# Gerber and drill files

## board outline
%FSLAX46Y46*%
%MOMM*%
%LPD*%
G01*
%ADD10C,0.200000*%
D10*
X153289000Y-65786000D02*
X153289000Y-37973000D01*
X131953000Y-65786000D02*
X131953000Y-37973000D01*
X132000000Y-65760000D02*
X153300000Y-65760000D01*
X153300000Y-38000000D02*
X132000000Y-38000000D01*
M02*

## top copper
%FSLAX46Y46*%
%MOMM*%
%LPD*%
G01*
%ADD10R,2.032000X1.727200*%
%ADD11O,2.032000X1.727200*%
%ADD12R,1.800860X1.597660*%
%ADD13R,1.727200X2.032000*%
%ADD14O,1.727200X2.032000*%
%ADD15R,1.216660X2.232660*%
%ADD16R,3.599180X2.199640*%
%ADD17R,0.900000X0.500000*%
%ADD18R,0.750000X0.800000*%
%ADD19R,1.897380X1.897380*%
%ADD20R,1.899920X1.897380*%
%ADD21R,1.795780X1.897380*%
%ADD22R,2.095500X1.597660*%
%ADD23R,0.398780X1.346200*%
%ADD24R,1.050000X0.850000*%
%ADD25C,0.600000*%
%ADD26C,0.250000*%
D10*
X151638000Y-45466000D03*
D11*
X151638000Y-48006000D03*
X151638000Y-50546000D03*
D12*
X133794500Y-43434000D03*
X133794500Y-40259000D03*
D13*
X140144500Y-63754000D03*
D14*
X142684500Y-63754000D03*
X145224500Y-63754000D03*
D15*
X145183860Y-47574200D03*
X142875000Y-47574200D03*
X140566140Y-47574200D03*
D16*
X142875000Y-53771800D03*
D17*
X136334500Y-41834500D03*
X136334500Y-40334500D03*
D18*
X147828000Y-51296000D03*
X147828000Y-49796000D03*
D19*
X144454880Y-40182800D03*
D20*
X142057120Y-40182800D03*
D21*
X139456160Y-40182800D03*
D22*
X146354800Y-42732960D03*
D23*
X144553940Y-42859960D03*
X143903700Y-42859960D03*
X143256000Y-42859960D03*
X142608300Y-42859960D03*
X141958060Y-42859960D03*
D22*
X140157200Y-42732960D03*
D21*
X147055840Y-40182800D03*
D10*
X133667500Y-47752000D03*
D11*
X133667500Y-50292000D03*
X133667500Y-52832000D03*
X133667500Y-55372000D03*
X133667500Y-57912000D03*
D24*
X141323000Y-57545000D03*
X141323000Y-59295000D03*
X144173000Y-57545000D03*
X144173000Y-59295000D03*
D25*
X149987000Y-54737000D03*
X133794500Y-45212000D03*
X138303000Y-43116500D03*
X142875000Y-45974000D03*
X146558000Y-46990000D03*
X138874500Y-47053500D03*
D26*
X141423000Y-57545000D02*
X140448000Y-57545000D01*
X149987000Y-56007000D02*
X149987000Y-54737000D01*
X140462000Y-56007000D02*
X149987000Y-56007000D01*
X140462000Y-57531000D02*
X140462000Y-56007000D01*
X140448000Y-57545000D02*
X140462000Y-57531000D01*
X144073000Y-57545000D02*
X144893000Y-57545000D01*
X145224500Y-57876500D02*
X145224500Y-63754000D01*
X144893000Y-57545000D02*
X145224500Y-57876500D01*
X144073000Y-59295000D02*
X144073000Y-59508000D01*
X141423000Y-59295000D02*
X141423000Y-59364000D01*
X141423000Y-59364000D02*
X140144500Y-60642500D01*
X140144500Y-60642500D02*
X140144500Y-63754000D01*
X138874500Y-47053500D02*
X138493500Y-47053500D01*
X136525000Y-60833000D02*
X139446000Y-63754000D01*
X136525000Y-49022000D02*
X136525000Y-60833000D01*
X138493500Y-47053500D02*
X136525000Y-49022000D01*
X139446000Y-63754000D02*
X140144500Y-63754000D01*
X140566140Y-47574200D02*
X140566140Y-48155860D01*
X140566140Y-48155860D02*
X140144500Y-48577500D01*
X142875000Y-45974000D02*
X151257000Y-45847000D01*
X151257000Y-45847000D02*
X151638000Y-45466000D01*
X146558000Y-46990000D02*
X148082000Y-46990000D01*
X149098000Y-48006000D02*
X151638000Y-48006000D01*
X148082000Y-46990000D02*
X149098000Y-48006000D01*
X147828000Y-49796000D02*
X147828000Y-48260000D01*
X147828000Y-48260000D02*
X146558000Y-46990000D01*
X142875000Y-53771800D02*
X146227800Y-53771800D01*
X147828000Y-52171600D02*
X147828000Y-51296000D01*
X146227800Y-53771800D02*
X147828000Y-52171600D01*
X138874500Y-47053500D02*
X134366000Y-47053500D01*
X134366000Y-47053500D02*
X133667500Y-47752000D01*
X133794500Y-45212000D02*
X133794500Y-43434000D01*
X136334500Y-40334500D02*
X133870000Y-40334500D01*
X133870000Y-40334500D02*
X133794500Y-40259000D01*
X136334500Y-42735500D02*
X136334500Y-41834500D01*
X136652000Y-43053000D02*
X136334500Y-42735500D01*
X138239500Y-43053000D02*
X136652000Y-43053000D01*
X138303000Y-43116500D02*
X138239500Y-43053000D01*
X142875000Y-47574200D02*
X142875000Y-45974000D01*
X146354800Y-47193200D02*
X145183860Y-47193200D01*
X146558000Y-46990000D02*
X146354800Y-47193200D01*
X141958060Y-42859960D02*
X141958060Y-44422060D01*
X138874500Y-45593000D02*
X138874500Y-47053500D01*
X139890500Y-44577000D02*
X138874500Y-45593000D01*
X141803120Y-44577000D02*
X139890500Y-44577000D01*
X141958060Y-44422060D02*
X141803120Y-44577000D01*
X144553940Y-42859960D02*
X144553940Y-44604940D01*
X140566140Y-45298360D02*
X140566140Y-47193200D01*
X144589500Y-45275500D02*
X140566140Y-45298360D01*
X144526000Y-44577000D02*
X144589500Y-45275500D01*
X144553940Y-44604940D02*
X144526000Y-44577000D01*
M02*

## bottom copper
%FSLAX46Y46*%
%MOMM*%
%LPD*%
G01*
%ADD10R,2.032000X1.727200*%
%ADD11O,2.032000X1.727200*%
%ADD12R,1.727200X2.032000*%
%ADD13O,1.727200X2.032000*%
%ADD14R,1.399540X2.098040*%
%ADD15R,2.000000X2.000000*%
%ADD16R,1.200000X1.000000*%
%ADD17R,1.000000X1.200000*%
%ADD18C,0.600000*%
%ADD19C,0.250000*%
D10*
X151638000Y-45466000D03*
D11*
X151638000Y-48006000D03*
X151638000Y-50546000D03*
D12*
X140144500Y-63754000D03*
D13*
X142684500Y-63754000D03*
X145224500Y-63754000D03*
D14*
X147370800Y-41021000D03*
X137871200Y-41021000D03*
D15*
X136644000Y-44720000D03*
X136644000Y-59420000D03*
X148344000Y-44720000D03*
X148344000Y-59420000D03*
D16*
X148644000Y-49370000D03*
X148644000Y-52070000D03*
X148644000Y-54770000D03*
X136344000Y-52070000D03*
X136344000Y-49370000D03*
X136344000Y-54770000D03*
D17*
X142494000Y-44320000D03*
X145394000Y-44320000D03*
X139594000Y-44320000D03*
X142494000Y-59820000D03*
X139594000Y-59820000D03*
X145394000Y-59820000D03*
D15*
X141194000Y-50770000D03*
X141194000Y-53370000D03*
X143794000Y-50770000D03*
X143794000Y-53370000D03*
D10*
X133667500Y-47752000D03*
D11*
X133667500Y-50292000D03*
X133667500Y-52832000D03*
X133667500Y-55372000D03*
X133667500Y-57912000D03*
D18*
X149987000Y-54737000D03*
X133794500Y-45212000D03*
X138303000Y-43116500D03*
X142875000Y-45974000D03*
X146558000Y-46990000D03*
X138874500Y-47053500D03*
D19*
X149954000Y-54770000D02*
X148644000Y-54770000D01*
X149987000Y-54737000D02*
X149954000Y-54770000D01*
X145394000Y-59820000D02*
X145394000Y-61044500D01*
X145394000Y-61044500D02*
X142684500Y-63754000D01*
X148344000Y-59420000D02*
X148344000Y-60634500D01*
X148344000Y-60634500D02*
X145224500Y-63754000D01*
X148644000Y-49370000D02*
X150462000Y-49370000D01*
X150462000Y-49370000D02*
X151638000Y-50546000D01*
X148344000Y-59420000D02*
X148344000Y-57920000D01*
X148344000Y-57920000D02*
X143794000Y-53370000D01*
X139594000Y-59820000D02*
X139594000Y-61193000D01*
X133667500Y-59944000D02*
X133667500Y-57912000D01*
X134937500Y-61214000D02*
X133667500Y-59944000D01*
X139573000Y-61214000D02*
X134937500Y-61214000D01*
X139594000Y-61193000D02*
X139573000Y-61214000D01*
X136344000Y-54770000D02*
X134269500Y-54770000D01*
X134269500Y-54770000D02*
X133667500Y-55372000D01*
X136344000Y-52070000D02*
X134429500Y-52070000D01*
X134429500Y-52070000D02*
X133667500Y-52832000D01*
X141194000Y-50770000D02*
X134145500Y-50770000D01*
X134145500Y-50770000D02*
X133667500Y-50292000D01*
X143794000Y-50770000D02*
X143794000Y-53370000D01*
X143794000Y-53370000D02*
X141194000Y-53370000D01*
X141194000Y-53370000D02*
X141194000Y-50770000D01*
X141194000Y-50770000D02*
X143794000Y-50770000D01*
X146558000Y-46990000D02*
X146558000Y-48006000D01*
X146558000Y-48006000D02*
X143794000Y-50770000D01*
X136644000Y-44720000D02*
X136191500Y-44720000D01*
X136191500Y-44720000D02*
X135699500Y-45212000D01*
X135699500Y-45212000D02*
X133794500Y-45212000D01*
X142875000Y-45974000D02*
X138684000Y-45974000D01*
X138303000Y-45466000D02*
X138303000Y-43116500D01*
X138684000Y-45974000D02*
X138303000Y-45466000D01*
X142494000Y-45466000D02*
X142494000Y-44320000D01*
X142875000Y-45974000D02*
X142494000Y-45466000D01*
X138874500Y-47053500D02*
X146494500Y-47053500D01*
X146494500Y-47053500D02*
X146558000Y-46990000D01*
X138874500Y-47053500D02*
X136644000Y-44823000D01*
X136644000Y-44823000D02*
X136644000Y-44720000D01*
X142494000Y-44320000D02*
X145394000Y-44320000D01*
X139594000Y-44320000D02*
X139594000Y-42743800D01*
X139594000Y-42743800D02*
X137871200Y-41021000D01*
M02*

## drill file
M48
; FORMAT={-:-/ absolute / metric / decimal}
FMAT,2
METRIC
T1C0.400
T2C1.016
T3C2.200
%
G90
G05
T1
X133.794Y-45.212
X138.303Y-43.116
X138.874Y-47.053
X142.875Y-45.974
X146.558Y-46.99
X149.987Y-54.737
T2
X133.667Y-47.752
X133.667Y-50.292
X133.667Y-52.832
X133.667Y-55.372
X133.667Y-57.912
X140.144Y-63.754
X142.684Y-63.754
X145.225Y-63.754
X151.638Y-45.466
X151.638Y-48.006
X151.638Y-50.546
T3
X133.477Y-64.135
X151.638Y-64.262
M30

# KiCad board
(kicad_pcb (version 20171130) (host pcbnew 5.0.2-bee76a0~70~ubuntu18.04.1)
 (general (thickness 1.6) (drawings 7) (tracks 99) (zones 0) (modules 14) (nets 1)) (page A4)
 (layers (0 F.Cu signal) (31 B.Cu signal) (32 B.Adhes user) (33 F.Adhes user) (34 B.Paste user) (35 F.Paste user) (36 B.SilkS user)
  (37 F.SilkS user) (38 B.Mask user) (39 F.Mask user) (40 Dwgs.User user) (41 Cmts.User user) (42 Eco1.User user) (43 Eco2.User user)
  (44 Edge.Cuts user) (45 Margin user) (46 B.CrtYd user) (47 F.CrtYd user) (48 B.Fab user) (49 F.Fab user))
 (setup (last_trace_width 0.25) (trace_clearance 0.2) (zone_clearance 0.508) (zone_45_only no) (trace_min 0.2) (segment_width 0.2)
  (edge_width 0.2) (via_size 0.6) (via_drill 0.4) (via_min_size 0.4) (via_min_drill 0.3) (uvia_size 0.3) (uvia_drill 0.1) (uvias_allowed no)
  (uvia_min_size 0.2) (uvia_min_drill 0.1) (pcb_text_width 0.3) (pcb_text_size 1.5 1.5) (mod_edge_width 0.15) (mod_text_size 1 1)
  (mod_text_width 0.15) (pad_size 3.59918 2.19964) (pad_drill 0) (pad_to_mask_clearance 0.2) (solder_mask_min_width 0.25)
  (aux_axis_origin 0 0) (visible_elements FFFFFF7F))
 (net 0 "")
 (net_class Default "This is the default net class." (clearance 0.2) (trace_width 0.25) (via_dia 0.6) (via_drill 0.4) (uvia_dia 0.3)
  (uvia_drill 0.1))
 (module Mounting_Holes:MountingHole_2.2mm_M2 (layer F.Cu) (at 133.477 64.135)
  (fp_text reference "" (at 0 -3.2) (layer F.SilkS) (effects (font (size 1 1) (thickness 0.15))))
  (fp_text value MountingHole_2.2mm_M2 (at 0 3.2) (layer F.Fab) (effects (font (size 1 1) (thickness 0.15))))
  (pad 1 np_thru_hole circle (at 0 0) (size 2.2 2.2) (drill 2.2) (layers *.Cu *.Mask F.SilkS)))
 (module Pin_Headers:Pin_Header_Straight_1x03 (layer F.Cu) (at 151.638 45.466)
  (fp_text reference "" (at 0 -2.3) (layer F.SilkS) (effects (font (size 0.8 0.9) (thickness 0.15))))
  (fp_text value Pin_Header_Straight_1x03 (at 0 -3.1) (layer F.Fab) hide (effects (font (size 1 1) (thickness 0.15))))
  (pad 1 thru_hole rect (at 0 0) (size 2.032 1.7272) (drill 1.016) (layers *.Cu *.Mask F.SilkS))
  (pad 2 thru_hole oval (at 0 2.54) (size 2.032 1.7272) (drill 1.016) (layers *.Cu *.Mask F.SilkS))
  (pad 3 thru_hole oval (at 0 5.08) (size 2.032 1.7272) (drill 1.016) (layers *.Cu *.Mask F.SilkS)))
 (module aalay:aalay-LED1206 (layer F.Cu) (at 133.7945 41.8465 90)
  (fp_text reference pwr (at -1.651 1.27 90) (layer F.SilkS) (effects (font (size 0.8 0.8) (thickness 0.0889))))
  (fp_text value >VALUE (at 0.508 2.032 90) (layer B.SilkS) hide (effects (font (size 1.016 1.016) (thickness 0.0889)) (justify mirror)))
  (pad A smd rect (at -1.5875 0 90) (size 1.59766 1.80086) (layers F.Cu F.Paste F.Mask))
  (pad K smd rect (at 1.5875 0 90) (size 1.59766 1.80086) (layers F.Cu F.Paste F.Mask)))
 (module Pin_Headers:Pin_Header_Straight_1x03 (layer F.Cu) (at 140.1445 63.754 90)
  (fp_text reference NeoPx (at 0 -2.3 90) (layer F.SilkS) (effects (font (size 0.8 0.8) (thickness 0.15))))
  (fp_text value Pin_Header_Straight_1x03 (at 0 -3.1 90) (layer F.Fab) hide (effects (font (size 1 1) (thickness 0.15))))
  (pad 1 thru_hole rect (at 0 0 90) (size 2.032 1.7272) (drill 1.016) (layers *.Cu *.Mask F.SilkS))
  (pad 2 thru_hole oval (at 0 2.54 90) (size 2.032 1.7272) (drill 1.016) (layers *.Cu *.Mask F.SilkS))
  (pad 3 thru_hole oval (at 0 5.08 90) (size 2.032 1.7272) (drill 1.016) (layers *.Cu *.Mask F.SilkS)))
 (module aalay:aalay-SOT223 (layer F.Cu) (at 142.875 50.673 180)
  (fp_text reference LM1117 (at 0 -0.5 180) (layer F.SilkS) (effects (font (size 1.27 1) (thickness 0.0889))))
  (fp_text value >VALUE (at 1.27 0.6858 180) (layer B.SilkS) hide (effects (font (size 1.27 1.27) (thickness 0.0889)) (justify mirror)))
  (pad GND smd rect (at -2.30886 3.0988 180) (size 1.21666 2.23266) (layers F.Cu F.Paste F.Mask))
  (pad OUT smd rect (at 0 3.0988 180) (size 1.21666 2.23266) (layers F.Cu F.Paste F.Mask))
  (pad IN smd rect (at 2.30886 3.0988 180) (size 1.21666 2.23266) (layers F.Cu F.Paste F.Mask))
  (pad OUT smd rect (at 0 -3.0988 180) (size 3.59918 2.19964) (layers F.Cu F.Paste F.Mask)))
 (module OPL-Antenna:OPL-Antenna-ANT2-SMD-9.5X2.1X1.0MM (layer B.Cu) (at 142.621 41.021 180)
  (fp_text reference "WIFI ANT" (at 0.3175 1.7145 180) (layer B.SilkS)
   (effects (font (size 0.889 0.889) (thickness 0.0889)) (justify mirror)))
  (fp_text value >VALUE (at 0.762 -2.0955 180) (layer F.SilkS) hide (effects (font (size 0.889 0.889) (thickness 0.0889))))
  (pad 1 smd rect (at -4.7498 0 180) (size 1.39954 2.09804) (layers B.Cu B.Paste B.Mask))
  (pad 2 smd rect (at 4.7498 0 180) (size 1.39954 2.09804) (layers B.Cu B.Paste B.Mask)))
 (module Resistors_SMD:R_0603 (layer F.Cu) (at 136.3345 41.0845 90)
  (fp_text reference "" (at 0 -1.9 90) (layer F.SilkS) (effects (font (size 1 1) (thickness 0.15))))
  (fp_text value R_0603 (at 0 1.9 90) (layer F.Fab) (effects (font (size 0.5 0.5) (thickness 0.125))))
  (pad 1 smd rect (at -0.75 0 90) (size 0.5 0.9) (layers F.Cu F.Paste F.Mask))
  (pad 2 smd rect (at 0.75 0 90) (size 0.5 0.9) (layers F.Cu F.Paste F.Mask)))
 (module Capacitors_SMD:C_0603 (layer F.Cu) (at 147.828 50.546 90)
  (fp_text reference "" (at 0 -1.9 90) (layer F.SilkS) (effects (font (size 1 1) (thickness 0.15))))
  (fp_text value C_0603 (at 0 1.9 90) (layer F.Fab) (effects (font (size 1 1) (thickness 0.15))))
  (pad 1 smd rect (at -0.75 0 90) (size 0.8 0.75) (layers F.Cu F.Paste F.Mask))
  (pad 2 smd rect (at 0.75 0 90) (size 0.8 0.75) (layers F.Cu F.Paste F.Mask)))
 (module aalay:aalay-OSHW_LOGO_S (layer F.Cu) (at 150.622 39.878)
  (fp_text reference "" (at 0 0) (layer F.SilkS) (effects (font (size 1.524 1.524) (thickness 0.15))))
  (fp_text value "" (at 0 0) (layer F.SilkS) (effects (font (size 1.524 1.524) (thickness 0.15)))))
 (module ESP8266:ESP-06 (layer B.Cu) (at 142.494 52.07 270)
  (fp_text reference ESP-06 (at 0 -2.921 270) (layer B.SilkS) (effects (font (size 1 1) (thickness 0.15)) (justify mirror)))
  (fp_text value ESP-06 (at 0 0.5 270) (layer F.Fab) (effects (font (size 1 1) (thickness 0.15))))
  (pad GND smd rect (at -7.35 5.85 270) (size 2 2) (layers B.Cu B.Paste B.Mask))
  (pad GP5 smd rect (at 7.35 5.85 270) (size 2 2) (layers B.Cu B.Paste B.Mask))
  (pad GP16 smd rect (at -7.35 -5.85 270) (size 2 2) (layers B.Cu B.Paste B.Mask))
  (pad GP15 smd rect (at 7.35 -5.85 270) (size 2 2) (layers B.Cu B.Paste B.Mask))
  (pad GP14 smd rect (at -2.7 -6.15 270) (size 1 1.2) (layers B.Cu B.Paste B.Mask))
  (pad GP12 smd rect (at 0 -6.15 270) (size 1 1.2) (layers B.Cu B.Paste B.Mask))
  (pad GP13 smd rect (at 2.7 -6.15 270) (size 1 1.2) (layers B.Cu B.Paste B.Mask))
  (pad TX smd rect (at 0 6.15 270) (size 1 1.2) (layers B.Cu B.Paste B.Mask))
  (pad RST smd rect (at -2.7 6.15 270) (size 1 1.2) (layers B.Cu B.Paste B.Mask))
  (pad RX smd rect (at 2.7 6.15 270) (size 1 1.2) (layers B.Cu B.Paste B.Mask))
  (pad 3.3 smd rect (at -7.75 0 270) (size 1.2 1) (layers B.Cu B.Paste B.Mask))
  (pad CHPD smd rect (at -7.75 -2.9 270) (size 1.2 1) (layers B.Cu B.Paste B.Mask))
  (pad ANT smd rect (at -7.75 2.9 270) (size 1.2 1) (layers B.Cu B.Paste B.Mask))
  (pad GP2 smd rect (at 7.75 0 270) (size 1.2 1) (layers B.Cu B.Paste B.Mask))
  (pad GP0 smd rect (at 7.75 2.9 270) (size 1.2 1) (layers B.Cu B.Paste B.Mask))
  (pad GP4 smd rect (at 7.75 -2.9 270) (size 1.2 1) (layers B.Cu B.Paste B.Mask))
  (pad GND smd rect (at -1.3 1.3 270) (size 2 2) (layers B.Cu B.Paste B.Mask))
  (pad GND smd rect (at 1.3 1.3 270) (size 2 2) (layers B.Cu B.Paste B.Mask))
  (pad GND smd rect (at -1.3 -1.3 270) (size 2 2) (layers B.Cu B.Paste B.Mask))
  (pad GND smd rect (at 1.3 -1.3 270) (size 2 2) (layers B.Cu B.Paste B.Mask)))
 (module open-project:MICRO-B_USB (layer F.Cu) (at 143.256 38.735 180)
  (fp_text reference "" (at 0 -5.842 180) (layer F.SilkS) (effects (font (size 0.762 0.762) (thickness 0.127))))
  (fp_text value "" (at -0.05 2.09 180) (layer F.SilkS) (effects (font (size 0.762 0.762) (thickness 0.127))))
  (pad "" smd rect (at -1.19888 -1.4478 180) (size 1.89738 1.89738) (layers F.Cu F.Paste F.Mask))
  (pad "" smd rect (at 1.19888 -1.4478 180) (size 1.89992 1.89738) (layers F.Cu F.Paste F.Mask))
  (pad "" smd rect (at 3.79984 -1.4478 180) (size 1.79578 1.89738) (layers F.Cu F.Paste F.Mask))
  (pad "" smd rect (at -3.0988 -3.99796 180) (size 2.0955 1.59766) (layers F.Cu F.Paste F.Mask))
  (pad 1 smd rect (at -1.29794 -4.12496 180) (size 0.39878 1.3462) (layers F.Cu F.Paste F.Mask) (clearance 0.2032))
  (pad 2 smd rect (at -0.6477 -4.12496 180) (size 0.39878 1.3462) (layers F.Cu F.Paste F.Mask) (clearance 0.2032))
  (pad 3 smd rect (at 0 -4.12496 180) (size 0.39878 1.3462) (layers F.Cu F.Paste F.Mask) (clearance 0.2032))
  (pad 4 smd rect (at 0.6477 -4.12496 180) (size 0.39878 1.3462) (layers F.Cu F.Paste F.Mask) (clearance 0.2032))
  (pad 5 smd rect (at 1.29794 -4.12496 180) (size 0.39878 1.3462) (layers F.Cu F.Paste F.Mask) (clearance 0.2032))
  (pad "" smd rect (at 3.0988 -3.99796 180) (size 2.0955 1.59766) (layers F.Cu F.Paste F.Mask))
  (pad "" smd rect (at -3.79984 -1.4478 180) (size 1.79578 1.89738) (layers F.Cu F.Paste F.Mask)))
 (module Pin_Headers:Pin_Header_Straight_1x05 (layer F.Cu) (at 133.6675 47.752)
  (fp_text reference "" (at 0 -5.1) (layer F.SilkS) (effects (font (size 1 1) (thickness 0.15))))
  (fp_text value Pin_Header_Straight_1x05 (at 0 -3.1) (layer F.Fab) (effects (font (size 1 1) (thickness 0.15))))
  (pad 1 thru_hole rect (at 0 0) (size 2.032 1.7272) (drill 1.016) (layers *.Cu *.Mask F.SilkS))
  (pad 2 thru_hole oval (at 0 2.54) (size 2.032 1.7272) (drill 1.016) (layers *.Cu *.Mask F.SilkS))
  (pad 3 thru_hole oval (at 0 5.08) (size 2.032 1.7272) (drill 1.016) (layers *.Cu *.Mask F.SilkS))
  (pad 4 thru_hole oval (at 0 7.62) (size 2.032 1.7272) (drill 1.016) (layers *.Cu *.Mask F.SilkS))
  (pad 5 thru_hole oval (at 0 10.16) (size 2.032 1.7272) (drill 1.016) (layers *.Cu *.Mask F.SilkS)))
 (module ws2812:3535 (layer F.Cu) (at 142.748 58.42 180)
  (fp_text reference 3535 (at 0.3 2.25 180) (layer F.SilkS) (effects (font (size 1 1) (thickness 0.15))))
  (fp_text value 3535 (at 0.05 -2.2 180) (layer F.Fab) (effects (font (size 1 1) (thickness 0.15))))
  (pad IN smd rect (at 1.325 0.875 180) (size 1.05 0.85) (drill (offset 0.1 0)) (layers F.Cu F.Paste F.Mask))
  (pad VDD smd rect (at 1.325 -0.875 180) (size 1.05 0.85) (drill (offset 0.1 0)) (layers F.Cu F.Paste F.Mask))
  (pad VSS smd rect (at -1.325 0.875 180) (size 1.05 0.85) (drill (offset -0.1 0)) (layers F.Cu F.Paste F.Mask))
  (pad OUT smd rect (at -1.325 -0.875 180) (size 1.05 0.85) (drill (offset -0.1 0)) (layers F.Cu F.Paste F.Mask)))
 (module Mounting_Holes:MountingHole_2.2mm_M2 (layer F.Cu) (at 151.638 64.262)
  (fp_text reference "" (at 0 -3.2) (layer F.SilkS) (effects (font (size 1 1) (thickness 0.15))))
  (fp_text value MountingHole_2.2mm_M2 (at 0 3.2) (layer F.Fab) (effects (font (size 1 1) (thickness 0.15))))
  (pad 1 np_thru_hole circle (at 0 0) (size 2.2 2.2) (drill 2.2) (layers *.Cu *.Mask F.SilkS)))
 (gr_line (start 153.289 65.786) (end 153.289 37.973) (angle 90) (layer Edge.Cuts) (width 0.2))
 (gr_line (start 131.953 65.786) (end 131.953 37.973) (angle 90) (layer Edge.Cuts) (width 0.2))
 (gr_line (start 132 65.76) (end 153.3 65.76) (angle 90) (layer Edge.Cuts) (width 0.2))
 (gr_line (start 153.3 38) (end 132 38) (angle 90) (layer Edge.Cuts) (width 0.2))
 (segment (start 141.423 57.545) (end 140.448 57.545) (width 0.25) (layer F.Cu) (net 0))
 (segment (start 149.954 54.77) (end 148.644 54.77) (width 0.25) (layer B.Cu) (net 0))
 (segment (start 149.987 54.737) (end 149.954 54.77) (width 0.25) (layer B.Cu) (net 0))
 (via (at 149.987 54.737) (size 0.6) (drill 0.4) (layers F.Cu B.Cu) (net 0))
 (segment (start 149.987 56.007) (end 149.987 54.737) (width 0.25) (layer F.Cu) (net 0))
 (segment (start 140.462 56.007) (end 149.987 56.007) (width 0.25) (layer F.Cu) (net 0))
 (segment (start 140.462 57.531) (end 140.462 56.007) (width 0.25) (layer F.Cu) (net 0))
 (segment (start 140.448 57.545) (end 140.462 57.531) (width 0.25) (layer F.Cu) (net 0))
 (segment (start 144.073 57.545) (end 144.893 57.545) (width 0.25) (layer F.Cu) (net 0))
 (segment (start 145.2245 57.8765) (end 145.2245 63.754) (width 0.25) (layer F.Cu) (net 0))
 (segment (start 144.893 57.545) (end 145.2245 57.8765) (width 0.25) (layer F.Cu) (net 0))
 (segment (start 144.073 59.295) (end 144.073 59.508) (width 0.25) (layer F.Cu) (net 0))
 (segment (start 141.423 59.295) (end 141.423 59.364) (width 0.25) (layer F.Cu) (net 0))
 (segment (start 141.423 59.364) (end 140.1445 60.6425) (width 0.25) (layer F.Cu) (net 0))
 (segment (start 140.1445 60.6425) (end 140.1445 63.754) (width 0.25) (layer F.Cu) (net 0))
 (segment (start 138.8745 47.0535) (end 138.4935 47.0535) (width 0.25) (layer F.Cu) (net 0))
 (segment (start 136.525 60.833) (end 139.446 63.754) (width 0.25) (layer F.Cu) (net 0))
 (segment (start 136.525 49.022) (end 136.525 60.833) (width 0.25) (layer F.Cu) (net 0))
 (segment (start 138.4935 47.0535) (end 136.525 49.022) (width 0.25) (layer F.Cu) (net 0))
 (segment (start 139.446 63.754) (end 140.1445 63.754) (width 0.25) (layer F.Cu) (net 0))
 (segment (start 140.56614 47.5742) (end 140.56614 48.15586) (width 0.25) (layer F.Cu) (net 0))
 (segment (start 140.56614 48.15586) (end 140.1445 48.5775) (width 0.25) (layer F.Cu) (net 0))
 (segment (start 145.394 59.82) (end 145.394 61.0445) (width 0.25) (layer B.Cu) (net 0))
 (segment (start 145.394 61.0445) (end 142.6845 63.754) (width 0.25) (layer B.Cu) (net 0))
 (segment (start 148.344 59.42) (end 148.344 60.6345) (width 0.25) (layer B.Cu) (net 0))
 (segment (start 148.344 60.6345) (end 145.2245 63.754) (width 0.25) (layer B.Cu) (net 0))
 (segment (start 148.644 49.37) (end 150.462 49.37) (width 0.25) (layer B.Cu) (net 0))
 (segment (start 150.462 49.37) (end 151.638 50.546) (width 0.25) (layer B.Cu) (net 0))
 (segment (start 142.875 45.974) (end 151.257 45.847) (width 0.25) (layer F.Cu) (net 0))
 (segment (start 151.257 45.847) (end 151.638 45.466) (width 0.25) (layer F.Cu) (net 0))
 (segment (start 146.558 46.99) (end 148.082 46.99) (width 0.25) (layer F.Cu) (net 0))
 (segment (start 149.098 48.006) (end 151.638 48.006) (width 0.25) (layer F.Cu) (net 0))
 (segment (start 148.082 46.99) (end 149.098 48.006) (width 0.25) (layer F.Cu) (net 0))
 (segment (start 147.828 49.796) (end 147.828 48.26) (width 0.25) (layer F.Cu) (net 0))
 (segment (start 147.828 48.26) (end 146.558 46.99) (width 0.25) (layer F.Cu) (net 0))
 (segment (start 142.875 53.7718) (end 146.2278 53.7718) (width 0.25) (layer F.Cu) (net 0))
 (segment (start 147.828 52.1716) (end 147.828 51.296) (width 0.25) (layer F.Cu) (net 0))
 (segment (start 146.2278 53.7718) (end 147.828 52.1716) (width 0.25) (layer F.Cu) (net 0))
 (segment (start 148.344 59.42) (end 148.344 57.92) (width 0.25) (layer B.Cu) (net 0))
 (segment (start 148.344 57.92) (end 143.794 53.37) (width 0.25) (layer B.Cu) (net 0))
 (segment (start 139.594 59.82) (end 139.594 61.193) (width 0.25) (layer B.Cu) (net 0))
 (segment (start 133.6675 59.944) (end 133.6675 57.912) (width 0.25) (layer B.Cu) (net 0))
 (segment (start 134.9375 61.214) (end 133.6675 59.944) (width 0.25) (layer B.Cu) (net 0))
 (segment (start 139.573 61.214) (end 134.9375 61.214) (width 0.25) (layer B.Cu) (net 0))
 (segment (start 139.594 61.193) (end 139.573 61.214) (width 0.25) (layer B.Cu) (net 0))
 (segment (start 136.344 54.77) (end 134.2695 54.77) (width 0.25) (layer B.Cu) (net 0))
 (segment (start 134.2695 54.77) (end 133.6675 55.372) (width 0.25) (layer B.Cu) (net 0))
 (segment (start 136.344 52.07) (end 134.4295 52.07) (width 0.25) (layer B.Cu) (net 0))
 (segment (start 134.4295 52.07) (end 133.6675 52.832) (width 0.25) (layer B.Cu) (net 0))
 (segment (start 141.194 50.77) (end 134.1455 50.77) (width 0.25) (layer B.Cu) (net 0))
 (segment (start 134.1455 50.77) (end 133.6675 50.292) (width 0.25) (layer B.Cu) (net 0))
 (segment (start 138.8745 47.0535) (end 134.366 47.0535) (width 0.25) (layer F.Cu) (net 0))
 (segment (start 134.366 47.0535) (end 133.6675 47.752) (width 0.25) (layer F.Cu) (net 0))
 (segment (start 143.794 50.77) (end 143.794 53.37) (width 0.25) (layer B.Cu) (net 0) (status 30))
 (segment (start 143.794 53.37) (end 141.194 53.37) (width 0.25) (layer B.Cu) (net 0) (status 30))
 (segment (start 141.194 53.37) (end 141.194 50.77) (width 0.25) (layer B.Cu) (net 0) (status 30))
 (segment (start 141.194 50.77) (end 143.794 50.77) (width 0.25) (layer B.Cu) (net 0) (status 30))
 (segment (start 146.558 46.99) (end 146.558 48.006) (width 0.25) (layer B.Cu) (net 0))
 (segment (start 146.558 48.006) (end 143.794 50.77) (width 0.25) (layer B.Cu) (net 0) (status 20))
 (segment (start 136.644 44.72) (end 136.1915 44.72) (width 0.25) (layer B.Cu) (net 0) (status 30))
 (segment (start 136.1915 44.72) (end 135.6995 45.212) (width 0.25) (layer B.Cu) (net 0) (status 30))
 (segment (start 135.6995 45.212) (end 133.7945 45.212) (width 0.25) (layer B.Cu) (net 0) (status 10))
 (via (at 133.7945 45.212) (size 0.6) (drill 0.4) (layers F.Cu B.Cu) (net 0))
 (segment (start 133.7945 45.212) (end 133.7945 43.434) (width 0.25) (layer F.Cu) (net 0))
 (segment (start 136.3345 40.3345) (end 133.87 40.3345) (width 0.25) (layer F.Cu) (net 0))
 (segment (start 133.87 40.3345) (end 133.7945 40.259) (width 0.25) (layer F.Cu) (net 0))
 (segment (start 142.875 45.974) (end 138.684 45.974) (width 0.25) (layer B.Cu) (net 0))
 (segment (start 136.3345 42.7355) (end 136.3345 41.8345) (width 0.25) (layer F.Cu) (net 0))
 (segment (start 136.652 43.053) (end 136.3345 42.7355) (width 0.25) (layer F.Cu) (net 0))
 (segment (start 138.2395 43.053) (end 136.652 43.053) (width 0.25) (layer F.Cu) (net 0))
 (segment (start 138.303 43.1165) (end 138.2395 43.053) (width 0.25) (layer F.Cu) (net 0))
 (via (at 138.303 43.1165) (size 0.6) (drill 0.4) (layers F.Cu B.Cu) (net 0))
 (segment (start 138.303 45.466) (end 138.303 43.1165) (width 0.25) (layer B.Cu) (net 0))
 (segment (start 138.684 45.974) (end 138.303 45.466) (width 0.25) (layer B.Cu) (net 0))
 (segment (start 142.875 47.5742) (end 142.875 45.974) (width 0.25) (layer F.Cu) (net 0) (status 10))
 (segment (start 142.494 45.466) (end 142.494 44.32) (width 0.25) (layer B.Cu) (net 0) (status 20))
 (segment (start 142.875 45.974) (end 142.494 45.466) (width 0.25) (layer B.Cu) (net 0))
 (via (at 142.875 45.974) (size 0.6) (drill 0.4) (layers F.Cu B.Cu) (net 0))
 (segment (start 138.8745 47.0535) (end 146.4945 47.0535) (width 0.25) (layer B.Cu) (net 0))
 (segment (start 146.3548 47.1932) (end 145.18386 47.1932) (width 0.25) (layer F.Cu) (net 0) (status 20))
 (segment (start 146.558 46.99) (end 146.3548 47.1932) (width 0.25) (layer F.Cu) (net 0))
 (via (at 146.558 46.99) (size 0.6) (drill 0.4) (layers F.Cu B.Cu) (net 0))
 (segment (start 146.4945 47.0535) (end 146.558 46.99) (width 0.25) (layer B.Cu) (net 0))
 (segment (start 141.95806 42.85996) (end 141.95806 44.42206) (width 0.25) (layer F.Cu) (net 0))
 (segment (start 138.8745 47.0535) (end 136.644 44.823) (width 0.25) (layer B.Cu) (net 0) (status 20))
 (via (at 138.8745 47.0535) (size 0.6) (drill 0.4) (layers F.Cu B.Cu) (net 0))
 (segment (start 138.8745 45.593) (end 138.8745 47.0535) (width 0.25) (layer F.Cu) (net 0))
 (segment (start 139.8905 44.577) (end 138.8745 45.593) (width 0.25) (layer F.Cu) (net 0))
 (segment (start 141.80312 44.577) (end 139.8905 44.577) (width 0.25) (layer F.Cu) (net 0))
 (segment (start 141.95806 44.42206) (end 141.80312 44.577) (width 0.25) (layer F.Cu) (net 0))
 (segment (start 136.644 44.823) (end 136.644 44.72) (width 0.25) (layer B.Cu) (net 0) (status 30))
 (segment (start 144.55394 42.85996) (end 144.55394 44.60494) (width 0.25) (layer F.Cu) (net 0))
 (segment (start 140.56614 45.29836) (end 140.56614 47.1932) (width 0.25) (layer F.Cu) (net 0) (status 20))
 (segment (start 144.5895 45.2755) (end 140.56614 45.29836) (width 0.25) (layer F.Cu) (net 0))
 (segment (start 144.526 44.577) (end 144.5895 45.2755) (width 0.25) (layer F.Cu) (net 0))
 (segment (start 144.55394 44.60494) (end 144.526 44.577) (width 0.25) (layer F.Cu) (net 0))
 (segment (start 142.494 44.32) (end 145.394 44.32) (width 0.25) (layer B.Cu) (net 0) (status 30))
 (segment (start 139.594 44.32) (end 139.594 42.7438) (width 0.25) (layer B.Cu) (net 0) (status 10))
 (segment (start 139.594 42.7438) (end 137.8712 41.021) (width 0.25) (layer B.Cu) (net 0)))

